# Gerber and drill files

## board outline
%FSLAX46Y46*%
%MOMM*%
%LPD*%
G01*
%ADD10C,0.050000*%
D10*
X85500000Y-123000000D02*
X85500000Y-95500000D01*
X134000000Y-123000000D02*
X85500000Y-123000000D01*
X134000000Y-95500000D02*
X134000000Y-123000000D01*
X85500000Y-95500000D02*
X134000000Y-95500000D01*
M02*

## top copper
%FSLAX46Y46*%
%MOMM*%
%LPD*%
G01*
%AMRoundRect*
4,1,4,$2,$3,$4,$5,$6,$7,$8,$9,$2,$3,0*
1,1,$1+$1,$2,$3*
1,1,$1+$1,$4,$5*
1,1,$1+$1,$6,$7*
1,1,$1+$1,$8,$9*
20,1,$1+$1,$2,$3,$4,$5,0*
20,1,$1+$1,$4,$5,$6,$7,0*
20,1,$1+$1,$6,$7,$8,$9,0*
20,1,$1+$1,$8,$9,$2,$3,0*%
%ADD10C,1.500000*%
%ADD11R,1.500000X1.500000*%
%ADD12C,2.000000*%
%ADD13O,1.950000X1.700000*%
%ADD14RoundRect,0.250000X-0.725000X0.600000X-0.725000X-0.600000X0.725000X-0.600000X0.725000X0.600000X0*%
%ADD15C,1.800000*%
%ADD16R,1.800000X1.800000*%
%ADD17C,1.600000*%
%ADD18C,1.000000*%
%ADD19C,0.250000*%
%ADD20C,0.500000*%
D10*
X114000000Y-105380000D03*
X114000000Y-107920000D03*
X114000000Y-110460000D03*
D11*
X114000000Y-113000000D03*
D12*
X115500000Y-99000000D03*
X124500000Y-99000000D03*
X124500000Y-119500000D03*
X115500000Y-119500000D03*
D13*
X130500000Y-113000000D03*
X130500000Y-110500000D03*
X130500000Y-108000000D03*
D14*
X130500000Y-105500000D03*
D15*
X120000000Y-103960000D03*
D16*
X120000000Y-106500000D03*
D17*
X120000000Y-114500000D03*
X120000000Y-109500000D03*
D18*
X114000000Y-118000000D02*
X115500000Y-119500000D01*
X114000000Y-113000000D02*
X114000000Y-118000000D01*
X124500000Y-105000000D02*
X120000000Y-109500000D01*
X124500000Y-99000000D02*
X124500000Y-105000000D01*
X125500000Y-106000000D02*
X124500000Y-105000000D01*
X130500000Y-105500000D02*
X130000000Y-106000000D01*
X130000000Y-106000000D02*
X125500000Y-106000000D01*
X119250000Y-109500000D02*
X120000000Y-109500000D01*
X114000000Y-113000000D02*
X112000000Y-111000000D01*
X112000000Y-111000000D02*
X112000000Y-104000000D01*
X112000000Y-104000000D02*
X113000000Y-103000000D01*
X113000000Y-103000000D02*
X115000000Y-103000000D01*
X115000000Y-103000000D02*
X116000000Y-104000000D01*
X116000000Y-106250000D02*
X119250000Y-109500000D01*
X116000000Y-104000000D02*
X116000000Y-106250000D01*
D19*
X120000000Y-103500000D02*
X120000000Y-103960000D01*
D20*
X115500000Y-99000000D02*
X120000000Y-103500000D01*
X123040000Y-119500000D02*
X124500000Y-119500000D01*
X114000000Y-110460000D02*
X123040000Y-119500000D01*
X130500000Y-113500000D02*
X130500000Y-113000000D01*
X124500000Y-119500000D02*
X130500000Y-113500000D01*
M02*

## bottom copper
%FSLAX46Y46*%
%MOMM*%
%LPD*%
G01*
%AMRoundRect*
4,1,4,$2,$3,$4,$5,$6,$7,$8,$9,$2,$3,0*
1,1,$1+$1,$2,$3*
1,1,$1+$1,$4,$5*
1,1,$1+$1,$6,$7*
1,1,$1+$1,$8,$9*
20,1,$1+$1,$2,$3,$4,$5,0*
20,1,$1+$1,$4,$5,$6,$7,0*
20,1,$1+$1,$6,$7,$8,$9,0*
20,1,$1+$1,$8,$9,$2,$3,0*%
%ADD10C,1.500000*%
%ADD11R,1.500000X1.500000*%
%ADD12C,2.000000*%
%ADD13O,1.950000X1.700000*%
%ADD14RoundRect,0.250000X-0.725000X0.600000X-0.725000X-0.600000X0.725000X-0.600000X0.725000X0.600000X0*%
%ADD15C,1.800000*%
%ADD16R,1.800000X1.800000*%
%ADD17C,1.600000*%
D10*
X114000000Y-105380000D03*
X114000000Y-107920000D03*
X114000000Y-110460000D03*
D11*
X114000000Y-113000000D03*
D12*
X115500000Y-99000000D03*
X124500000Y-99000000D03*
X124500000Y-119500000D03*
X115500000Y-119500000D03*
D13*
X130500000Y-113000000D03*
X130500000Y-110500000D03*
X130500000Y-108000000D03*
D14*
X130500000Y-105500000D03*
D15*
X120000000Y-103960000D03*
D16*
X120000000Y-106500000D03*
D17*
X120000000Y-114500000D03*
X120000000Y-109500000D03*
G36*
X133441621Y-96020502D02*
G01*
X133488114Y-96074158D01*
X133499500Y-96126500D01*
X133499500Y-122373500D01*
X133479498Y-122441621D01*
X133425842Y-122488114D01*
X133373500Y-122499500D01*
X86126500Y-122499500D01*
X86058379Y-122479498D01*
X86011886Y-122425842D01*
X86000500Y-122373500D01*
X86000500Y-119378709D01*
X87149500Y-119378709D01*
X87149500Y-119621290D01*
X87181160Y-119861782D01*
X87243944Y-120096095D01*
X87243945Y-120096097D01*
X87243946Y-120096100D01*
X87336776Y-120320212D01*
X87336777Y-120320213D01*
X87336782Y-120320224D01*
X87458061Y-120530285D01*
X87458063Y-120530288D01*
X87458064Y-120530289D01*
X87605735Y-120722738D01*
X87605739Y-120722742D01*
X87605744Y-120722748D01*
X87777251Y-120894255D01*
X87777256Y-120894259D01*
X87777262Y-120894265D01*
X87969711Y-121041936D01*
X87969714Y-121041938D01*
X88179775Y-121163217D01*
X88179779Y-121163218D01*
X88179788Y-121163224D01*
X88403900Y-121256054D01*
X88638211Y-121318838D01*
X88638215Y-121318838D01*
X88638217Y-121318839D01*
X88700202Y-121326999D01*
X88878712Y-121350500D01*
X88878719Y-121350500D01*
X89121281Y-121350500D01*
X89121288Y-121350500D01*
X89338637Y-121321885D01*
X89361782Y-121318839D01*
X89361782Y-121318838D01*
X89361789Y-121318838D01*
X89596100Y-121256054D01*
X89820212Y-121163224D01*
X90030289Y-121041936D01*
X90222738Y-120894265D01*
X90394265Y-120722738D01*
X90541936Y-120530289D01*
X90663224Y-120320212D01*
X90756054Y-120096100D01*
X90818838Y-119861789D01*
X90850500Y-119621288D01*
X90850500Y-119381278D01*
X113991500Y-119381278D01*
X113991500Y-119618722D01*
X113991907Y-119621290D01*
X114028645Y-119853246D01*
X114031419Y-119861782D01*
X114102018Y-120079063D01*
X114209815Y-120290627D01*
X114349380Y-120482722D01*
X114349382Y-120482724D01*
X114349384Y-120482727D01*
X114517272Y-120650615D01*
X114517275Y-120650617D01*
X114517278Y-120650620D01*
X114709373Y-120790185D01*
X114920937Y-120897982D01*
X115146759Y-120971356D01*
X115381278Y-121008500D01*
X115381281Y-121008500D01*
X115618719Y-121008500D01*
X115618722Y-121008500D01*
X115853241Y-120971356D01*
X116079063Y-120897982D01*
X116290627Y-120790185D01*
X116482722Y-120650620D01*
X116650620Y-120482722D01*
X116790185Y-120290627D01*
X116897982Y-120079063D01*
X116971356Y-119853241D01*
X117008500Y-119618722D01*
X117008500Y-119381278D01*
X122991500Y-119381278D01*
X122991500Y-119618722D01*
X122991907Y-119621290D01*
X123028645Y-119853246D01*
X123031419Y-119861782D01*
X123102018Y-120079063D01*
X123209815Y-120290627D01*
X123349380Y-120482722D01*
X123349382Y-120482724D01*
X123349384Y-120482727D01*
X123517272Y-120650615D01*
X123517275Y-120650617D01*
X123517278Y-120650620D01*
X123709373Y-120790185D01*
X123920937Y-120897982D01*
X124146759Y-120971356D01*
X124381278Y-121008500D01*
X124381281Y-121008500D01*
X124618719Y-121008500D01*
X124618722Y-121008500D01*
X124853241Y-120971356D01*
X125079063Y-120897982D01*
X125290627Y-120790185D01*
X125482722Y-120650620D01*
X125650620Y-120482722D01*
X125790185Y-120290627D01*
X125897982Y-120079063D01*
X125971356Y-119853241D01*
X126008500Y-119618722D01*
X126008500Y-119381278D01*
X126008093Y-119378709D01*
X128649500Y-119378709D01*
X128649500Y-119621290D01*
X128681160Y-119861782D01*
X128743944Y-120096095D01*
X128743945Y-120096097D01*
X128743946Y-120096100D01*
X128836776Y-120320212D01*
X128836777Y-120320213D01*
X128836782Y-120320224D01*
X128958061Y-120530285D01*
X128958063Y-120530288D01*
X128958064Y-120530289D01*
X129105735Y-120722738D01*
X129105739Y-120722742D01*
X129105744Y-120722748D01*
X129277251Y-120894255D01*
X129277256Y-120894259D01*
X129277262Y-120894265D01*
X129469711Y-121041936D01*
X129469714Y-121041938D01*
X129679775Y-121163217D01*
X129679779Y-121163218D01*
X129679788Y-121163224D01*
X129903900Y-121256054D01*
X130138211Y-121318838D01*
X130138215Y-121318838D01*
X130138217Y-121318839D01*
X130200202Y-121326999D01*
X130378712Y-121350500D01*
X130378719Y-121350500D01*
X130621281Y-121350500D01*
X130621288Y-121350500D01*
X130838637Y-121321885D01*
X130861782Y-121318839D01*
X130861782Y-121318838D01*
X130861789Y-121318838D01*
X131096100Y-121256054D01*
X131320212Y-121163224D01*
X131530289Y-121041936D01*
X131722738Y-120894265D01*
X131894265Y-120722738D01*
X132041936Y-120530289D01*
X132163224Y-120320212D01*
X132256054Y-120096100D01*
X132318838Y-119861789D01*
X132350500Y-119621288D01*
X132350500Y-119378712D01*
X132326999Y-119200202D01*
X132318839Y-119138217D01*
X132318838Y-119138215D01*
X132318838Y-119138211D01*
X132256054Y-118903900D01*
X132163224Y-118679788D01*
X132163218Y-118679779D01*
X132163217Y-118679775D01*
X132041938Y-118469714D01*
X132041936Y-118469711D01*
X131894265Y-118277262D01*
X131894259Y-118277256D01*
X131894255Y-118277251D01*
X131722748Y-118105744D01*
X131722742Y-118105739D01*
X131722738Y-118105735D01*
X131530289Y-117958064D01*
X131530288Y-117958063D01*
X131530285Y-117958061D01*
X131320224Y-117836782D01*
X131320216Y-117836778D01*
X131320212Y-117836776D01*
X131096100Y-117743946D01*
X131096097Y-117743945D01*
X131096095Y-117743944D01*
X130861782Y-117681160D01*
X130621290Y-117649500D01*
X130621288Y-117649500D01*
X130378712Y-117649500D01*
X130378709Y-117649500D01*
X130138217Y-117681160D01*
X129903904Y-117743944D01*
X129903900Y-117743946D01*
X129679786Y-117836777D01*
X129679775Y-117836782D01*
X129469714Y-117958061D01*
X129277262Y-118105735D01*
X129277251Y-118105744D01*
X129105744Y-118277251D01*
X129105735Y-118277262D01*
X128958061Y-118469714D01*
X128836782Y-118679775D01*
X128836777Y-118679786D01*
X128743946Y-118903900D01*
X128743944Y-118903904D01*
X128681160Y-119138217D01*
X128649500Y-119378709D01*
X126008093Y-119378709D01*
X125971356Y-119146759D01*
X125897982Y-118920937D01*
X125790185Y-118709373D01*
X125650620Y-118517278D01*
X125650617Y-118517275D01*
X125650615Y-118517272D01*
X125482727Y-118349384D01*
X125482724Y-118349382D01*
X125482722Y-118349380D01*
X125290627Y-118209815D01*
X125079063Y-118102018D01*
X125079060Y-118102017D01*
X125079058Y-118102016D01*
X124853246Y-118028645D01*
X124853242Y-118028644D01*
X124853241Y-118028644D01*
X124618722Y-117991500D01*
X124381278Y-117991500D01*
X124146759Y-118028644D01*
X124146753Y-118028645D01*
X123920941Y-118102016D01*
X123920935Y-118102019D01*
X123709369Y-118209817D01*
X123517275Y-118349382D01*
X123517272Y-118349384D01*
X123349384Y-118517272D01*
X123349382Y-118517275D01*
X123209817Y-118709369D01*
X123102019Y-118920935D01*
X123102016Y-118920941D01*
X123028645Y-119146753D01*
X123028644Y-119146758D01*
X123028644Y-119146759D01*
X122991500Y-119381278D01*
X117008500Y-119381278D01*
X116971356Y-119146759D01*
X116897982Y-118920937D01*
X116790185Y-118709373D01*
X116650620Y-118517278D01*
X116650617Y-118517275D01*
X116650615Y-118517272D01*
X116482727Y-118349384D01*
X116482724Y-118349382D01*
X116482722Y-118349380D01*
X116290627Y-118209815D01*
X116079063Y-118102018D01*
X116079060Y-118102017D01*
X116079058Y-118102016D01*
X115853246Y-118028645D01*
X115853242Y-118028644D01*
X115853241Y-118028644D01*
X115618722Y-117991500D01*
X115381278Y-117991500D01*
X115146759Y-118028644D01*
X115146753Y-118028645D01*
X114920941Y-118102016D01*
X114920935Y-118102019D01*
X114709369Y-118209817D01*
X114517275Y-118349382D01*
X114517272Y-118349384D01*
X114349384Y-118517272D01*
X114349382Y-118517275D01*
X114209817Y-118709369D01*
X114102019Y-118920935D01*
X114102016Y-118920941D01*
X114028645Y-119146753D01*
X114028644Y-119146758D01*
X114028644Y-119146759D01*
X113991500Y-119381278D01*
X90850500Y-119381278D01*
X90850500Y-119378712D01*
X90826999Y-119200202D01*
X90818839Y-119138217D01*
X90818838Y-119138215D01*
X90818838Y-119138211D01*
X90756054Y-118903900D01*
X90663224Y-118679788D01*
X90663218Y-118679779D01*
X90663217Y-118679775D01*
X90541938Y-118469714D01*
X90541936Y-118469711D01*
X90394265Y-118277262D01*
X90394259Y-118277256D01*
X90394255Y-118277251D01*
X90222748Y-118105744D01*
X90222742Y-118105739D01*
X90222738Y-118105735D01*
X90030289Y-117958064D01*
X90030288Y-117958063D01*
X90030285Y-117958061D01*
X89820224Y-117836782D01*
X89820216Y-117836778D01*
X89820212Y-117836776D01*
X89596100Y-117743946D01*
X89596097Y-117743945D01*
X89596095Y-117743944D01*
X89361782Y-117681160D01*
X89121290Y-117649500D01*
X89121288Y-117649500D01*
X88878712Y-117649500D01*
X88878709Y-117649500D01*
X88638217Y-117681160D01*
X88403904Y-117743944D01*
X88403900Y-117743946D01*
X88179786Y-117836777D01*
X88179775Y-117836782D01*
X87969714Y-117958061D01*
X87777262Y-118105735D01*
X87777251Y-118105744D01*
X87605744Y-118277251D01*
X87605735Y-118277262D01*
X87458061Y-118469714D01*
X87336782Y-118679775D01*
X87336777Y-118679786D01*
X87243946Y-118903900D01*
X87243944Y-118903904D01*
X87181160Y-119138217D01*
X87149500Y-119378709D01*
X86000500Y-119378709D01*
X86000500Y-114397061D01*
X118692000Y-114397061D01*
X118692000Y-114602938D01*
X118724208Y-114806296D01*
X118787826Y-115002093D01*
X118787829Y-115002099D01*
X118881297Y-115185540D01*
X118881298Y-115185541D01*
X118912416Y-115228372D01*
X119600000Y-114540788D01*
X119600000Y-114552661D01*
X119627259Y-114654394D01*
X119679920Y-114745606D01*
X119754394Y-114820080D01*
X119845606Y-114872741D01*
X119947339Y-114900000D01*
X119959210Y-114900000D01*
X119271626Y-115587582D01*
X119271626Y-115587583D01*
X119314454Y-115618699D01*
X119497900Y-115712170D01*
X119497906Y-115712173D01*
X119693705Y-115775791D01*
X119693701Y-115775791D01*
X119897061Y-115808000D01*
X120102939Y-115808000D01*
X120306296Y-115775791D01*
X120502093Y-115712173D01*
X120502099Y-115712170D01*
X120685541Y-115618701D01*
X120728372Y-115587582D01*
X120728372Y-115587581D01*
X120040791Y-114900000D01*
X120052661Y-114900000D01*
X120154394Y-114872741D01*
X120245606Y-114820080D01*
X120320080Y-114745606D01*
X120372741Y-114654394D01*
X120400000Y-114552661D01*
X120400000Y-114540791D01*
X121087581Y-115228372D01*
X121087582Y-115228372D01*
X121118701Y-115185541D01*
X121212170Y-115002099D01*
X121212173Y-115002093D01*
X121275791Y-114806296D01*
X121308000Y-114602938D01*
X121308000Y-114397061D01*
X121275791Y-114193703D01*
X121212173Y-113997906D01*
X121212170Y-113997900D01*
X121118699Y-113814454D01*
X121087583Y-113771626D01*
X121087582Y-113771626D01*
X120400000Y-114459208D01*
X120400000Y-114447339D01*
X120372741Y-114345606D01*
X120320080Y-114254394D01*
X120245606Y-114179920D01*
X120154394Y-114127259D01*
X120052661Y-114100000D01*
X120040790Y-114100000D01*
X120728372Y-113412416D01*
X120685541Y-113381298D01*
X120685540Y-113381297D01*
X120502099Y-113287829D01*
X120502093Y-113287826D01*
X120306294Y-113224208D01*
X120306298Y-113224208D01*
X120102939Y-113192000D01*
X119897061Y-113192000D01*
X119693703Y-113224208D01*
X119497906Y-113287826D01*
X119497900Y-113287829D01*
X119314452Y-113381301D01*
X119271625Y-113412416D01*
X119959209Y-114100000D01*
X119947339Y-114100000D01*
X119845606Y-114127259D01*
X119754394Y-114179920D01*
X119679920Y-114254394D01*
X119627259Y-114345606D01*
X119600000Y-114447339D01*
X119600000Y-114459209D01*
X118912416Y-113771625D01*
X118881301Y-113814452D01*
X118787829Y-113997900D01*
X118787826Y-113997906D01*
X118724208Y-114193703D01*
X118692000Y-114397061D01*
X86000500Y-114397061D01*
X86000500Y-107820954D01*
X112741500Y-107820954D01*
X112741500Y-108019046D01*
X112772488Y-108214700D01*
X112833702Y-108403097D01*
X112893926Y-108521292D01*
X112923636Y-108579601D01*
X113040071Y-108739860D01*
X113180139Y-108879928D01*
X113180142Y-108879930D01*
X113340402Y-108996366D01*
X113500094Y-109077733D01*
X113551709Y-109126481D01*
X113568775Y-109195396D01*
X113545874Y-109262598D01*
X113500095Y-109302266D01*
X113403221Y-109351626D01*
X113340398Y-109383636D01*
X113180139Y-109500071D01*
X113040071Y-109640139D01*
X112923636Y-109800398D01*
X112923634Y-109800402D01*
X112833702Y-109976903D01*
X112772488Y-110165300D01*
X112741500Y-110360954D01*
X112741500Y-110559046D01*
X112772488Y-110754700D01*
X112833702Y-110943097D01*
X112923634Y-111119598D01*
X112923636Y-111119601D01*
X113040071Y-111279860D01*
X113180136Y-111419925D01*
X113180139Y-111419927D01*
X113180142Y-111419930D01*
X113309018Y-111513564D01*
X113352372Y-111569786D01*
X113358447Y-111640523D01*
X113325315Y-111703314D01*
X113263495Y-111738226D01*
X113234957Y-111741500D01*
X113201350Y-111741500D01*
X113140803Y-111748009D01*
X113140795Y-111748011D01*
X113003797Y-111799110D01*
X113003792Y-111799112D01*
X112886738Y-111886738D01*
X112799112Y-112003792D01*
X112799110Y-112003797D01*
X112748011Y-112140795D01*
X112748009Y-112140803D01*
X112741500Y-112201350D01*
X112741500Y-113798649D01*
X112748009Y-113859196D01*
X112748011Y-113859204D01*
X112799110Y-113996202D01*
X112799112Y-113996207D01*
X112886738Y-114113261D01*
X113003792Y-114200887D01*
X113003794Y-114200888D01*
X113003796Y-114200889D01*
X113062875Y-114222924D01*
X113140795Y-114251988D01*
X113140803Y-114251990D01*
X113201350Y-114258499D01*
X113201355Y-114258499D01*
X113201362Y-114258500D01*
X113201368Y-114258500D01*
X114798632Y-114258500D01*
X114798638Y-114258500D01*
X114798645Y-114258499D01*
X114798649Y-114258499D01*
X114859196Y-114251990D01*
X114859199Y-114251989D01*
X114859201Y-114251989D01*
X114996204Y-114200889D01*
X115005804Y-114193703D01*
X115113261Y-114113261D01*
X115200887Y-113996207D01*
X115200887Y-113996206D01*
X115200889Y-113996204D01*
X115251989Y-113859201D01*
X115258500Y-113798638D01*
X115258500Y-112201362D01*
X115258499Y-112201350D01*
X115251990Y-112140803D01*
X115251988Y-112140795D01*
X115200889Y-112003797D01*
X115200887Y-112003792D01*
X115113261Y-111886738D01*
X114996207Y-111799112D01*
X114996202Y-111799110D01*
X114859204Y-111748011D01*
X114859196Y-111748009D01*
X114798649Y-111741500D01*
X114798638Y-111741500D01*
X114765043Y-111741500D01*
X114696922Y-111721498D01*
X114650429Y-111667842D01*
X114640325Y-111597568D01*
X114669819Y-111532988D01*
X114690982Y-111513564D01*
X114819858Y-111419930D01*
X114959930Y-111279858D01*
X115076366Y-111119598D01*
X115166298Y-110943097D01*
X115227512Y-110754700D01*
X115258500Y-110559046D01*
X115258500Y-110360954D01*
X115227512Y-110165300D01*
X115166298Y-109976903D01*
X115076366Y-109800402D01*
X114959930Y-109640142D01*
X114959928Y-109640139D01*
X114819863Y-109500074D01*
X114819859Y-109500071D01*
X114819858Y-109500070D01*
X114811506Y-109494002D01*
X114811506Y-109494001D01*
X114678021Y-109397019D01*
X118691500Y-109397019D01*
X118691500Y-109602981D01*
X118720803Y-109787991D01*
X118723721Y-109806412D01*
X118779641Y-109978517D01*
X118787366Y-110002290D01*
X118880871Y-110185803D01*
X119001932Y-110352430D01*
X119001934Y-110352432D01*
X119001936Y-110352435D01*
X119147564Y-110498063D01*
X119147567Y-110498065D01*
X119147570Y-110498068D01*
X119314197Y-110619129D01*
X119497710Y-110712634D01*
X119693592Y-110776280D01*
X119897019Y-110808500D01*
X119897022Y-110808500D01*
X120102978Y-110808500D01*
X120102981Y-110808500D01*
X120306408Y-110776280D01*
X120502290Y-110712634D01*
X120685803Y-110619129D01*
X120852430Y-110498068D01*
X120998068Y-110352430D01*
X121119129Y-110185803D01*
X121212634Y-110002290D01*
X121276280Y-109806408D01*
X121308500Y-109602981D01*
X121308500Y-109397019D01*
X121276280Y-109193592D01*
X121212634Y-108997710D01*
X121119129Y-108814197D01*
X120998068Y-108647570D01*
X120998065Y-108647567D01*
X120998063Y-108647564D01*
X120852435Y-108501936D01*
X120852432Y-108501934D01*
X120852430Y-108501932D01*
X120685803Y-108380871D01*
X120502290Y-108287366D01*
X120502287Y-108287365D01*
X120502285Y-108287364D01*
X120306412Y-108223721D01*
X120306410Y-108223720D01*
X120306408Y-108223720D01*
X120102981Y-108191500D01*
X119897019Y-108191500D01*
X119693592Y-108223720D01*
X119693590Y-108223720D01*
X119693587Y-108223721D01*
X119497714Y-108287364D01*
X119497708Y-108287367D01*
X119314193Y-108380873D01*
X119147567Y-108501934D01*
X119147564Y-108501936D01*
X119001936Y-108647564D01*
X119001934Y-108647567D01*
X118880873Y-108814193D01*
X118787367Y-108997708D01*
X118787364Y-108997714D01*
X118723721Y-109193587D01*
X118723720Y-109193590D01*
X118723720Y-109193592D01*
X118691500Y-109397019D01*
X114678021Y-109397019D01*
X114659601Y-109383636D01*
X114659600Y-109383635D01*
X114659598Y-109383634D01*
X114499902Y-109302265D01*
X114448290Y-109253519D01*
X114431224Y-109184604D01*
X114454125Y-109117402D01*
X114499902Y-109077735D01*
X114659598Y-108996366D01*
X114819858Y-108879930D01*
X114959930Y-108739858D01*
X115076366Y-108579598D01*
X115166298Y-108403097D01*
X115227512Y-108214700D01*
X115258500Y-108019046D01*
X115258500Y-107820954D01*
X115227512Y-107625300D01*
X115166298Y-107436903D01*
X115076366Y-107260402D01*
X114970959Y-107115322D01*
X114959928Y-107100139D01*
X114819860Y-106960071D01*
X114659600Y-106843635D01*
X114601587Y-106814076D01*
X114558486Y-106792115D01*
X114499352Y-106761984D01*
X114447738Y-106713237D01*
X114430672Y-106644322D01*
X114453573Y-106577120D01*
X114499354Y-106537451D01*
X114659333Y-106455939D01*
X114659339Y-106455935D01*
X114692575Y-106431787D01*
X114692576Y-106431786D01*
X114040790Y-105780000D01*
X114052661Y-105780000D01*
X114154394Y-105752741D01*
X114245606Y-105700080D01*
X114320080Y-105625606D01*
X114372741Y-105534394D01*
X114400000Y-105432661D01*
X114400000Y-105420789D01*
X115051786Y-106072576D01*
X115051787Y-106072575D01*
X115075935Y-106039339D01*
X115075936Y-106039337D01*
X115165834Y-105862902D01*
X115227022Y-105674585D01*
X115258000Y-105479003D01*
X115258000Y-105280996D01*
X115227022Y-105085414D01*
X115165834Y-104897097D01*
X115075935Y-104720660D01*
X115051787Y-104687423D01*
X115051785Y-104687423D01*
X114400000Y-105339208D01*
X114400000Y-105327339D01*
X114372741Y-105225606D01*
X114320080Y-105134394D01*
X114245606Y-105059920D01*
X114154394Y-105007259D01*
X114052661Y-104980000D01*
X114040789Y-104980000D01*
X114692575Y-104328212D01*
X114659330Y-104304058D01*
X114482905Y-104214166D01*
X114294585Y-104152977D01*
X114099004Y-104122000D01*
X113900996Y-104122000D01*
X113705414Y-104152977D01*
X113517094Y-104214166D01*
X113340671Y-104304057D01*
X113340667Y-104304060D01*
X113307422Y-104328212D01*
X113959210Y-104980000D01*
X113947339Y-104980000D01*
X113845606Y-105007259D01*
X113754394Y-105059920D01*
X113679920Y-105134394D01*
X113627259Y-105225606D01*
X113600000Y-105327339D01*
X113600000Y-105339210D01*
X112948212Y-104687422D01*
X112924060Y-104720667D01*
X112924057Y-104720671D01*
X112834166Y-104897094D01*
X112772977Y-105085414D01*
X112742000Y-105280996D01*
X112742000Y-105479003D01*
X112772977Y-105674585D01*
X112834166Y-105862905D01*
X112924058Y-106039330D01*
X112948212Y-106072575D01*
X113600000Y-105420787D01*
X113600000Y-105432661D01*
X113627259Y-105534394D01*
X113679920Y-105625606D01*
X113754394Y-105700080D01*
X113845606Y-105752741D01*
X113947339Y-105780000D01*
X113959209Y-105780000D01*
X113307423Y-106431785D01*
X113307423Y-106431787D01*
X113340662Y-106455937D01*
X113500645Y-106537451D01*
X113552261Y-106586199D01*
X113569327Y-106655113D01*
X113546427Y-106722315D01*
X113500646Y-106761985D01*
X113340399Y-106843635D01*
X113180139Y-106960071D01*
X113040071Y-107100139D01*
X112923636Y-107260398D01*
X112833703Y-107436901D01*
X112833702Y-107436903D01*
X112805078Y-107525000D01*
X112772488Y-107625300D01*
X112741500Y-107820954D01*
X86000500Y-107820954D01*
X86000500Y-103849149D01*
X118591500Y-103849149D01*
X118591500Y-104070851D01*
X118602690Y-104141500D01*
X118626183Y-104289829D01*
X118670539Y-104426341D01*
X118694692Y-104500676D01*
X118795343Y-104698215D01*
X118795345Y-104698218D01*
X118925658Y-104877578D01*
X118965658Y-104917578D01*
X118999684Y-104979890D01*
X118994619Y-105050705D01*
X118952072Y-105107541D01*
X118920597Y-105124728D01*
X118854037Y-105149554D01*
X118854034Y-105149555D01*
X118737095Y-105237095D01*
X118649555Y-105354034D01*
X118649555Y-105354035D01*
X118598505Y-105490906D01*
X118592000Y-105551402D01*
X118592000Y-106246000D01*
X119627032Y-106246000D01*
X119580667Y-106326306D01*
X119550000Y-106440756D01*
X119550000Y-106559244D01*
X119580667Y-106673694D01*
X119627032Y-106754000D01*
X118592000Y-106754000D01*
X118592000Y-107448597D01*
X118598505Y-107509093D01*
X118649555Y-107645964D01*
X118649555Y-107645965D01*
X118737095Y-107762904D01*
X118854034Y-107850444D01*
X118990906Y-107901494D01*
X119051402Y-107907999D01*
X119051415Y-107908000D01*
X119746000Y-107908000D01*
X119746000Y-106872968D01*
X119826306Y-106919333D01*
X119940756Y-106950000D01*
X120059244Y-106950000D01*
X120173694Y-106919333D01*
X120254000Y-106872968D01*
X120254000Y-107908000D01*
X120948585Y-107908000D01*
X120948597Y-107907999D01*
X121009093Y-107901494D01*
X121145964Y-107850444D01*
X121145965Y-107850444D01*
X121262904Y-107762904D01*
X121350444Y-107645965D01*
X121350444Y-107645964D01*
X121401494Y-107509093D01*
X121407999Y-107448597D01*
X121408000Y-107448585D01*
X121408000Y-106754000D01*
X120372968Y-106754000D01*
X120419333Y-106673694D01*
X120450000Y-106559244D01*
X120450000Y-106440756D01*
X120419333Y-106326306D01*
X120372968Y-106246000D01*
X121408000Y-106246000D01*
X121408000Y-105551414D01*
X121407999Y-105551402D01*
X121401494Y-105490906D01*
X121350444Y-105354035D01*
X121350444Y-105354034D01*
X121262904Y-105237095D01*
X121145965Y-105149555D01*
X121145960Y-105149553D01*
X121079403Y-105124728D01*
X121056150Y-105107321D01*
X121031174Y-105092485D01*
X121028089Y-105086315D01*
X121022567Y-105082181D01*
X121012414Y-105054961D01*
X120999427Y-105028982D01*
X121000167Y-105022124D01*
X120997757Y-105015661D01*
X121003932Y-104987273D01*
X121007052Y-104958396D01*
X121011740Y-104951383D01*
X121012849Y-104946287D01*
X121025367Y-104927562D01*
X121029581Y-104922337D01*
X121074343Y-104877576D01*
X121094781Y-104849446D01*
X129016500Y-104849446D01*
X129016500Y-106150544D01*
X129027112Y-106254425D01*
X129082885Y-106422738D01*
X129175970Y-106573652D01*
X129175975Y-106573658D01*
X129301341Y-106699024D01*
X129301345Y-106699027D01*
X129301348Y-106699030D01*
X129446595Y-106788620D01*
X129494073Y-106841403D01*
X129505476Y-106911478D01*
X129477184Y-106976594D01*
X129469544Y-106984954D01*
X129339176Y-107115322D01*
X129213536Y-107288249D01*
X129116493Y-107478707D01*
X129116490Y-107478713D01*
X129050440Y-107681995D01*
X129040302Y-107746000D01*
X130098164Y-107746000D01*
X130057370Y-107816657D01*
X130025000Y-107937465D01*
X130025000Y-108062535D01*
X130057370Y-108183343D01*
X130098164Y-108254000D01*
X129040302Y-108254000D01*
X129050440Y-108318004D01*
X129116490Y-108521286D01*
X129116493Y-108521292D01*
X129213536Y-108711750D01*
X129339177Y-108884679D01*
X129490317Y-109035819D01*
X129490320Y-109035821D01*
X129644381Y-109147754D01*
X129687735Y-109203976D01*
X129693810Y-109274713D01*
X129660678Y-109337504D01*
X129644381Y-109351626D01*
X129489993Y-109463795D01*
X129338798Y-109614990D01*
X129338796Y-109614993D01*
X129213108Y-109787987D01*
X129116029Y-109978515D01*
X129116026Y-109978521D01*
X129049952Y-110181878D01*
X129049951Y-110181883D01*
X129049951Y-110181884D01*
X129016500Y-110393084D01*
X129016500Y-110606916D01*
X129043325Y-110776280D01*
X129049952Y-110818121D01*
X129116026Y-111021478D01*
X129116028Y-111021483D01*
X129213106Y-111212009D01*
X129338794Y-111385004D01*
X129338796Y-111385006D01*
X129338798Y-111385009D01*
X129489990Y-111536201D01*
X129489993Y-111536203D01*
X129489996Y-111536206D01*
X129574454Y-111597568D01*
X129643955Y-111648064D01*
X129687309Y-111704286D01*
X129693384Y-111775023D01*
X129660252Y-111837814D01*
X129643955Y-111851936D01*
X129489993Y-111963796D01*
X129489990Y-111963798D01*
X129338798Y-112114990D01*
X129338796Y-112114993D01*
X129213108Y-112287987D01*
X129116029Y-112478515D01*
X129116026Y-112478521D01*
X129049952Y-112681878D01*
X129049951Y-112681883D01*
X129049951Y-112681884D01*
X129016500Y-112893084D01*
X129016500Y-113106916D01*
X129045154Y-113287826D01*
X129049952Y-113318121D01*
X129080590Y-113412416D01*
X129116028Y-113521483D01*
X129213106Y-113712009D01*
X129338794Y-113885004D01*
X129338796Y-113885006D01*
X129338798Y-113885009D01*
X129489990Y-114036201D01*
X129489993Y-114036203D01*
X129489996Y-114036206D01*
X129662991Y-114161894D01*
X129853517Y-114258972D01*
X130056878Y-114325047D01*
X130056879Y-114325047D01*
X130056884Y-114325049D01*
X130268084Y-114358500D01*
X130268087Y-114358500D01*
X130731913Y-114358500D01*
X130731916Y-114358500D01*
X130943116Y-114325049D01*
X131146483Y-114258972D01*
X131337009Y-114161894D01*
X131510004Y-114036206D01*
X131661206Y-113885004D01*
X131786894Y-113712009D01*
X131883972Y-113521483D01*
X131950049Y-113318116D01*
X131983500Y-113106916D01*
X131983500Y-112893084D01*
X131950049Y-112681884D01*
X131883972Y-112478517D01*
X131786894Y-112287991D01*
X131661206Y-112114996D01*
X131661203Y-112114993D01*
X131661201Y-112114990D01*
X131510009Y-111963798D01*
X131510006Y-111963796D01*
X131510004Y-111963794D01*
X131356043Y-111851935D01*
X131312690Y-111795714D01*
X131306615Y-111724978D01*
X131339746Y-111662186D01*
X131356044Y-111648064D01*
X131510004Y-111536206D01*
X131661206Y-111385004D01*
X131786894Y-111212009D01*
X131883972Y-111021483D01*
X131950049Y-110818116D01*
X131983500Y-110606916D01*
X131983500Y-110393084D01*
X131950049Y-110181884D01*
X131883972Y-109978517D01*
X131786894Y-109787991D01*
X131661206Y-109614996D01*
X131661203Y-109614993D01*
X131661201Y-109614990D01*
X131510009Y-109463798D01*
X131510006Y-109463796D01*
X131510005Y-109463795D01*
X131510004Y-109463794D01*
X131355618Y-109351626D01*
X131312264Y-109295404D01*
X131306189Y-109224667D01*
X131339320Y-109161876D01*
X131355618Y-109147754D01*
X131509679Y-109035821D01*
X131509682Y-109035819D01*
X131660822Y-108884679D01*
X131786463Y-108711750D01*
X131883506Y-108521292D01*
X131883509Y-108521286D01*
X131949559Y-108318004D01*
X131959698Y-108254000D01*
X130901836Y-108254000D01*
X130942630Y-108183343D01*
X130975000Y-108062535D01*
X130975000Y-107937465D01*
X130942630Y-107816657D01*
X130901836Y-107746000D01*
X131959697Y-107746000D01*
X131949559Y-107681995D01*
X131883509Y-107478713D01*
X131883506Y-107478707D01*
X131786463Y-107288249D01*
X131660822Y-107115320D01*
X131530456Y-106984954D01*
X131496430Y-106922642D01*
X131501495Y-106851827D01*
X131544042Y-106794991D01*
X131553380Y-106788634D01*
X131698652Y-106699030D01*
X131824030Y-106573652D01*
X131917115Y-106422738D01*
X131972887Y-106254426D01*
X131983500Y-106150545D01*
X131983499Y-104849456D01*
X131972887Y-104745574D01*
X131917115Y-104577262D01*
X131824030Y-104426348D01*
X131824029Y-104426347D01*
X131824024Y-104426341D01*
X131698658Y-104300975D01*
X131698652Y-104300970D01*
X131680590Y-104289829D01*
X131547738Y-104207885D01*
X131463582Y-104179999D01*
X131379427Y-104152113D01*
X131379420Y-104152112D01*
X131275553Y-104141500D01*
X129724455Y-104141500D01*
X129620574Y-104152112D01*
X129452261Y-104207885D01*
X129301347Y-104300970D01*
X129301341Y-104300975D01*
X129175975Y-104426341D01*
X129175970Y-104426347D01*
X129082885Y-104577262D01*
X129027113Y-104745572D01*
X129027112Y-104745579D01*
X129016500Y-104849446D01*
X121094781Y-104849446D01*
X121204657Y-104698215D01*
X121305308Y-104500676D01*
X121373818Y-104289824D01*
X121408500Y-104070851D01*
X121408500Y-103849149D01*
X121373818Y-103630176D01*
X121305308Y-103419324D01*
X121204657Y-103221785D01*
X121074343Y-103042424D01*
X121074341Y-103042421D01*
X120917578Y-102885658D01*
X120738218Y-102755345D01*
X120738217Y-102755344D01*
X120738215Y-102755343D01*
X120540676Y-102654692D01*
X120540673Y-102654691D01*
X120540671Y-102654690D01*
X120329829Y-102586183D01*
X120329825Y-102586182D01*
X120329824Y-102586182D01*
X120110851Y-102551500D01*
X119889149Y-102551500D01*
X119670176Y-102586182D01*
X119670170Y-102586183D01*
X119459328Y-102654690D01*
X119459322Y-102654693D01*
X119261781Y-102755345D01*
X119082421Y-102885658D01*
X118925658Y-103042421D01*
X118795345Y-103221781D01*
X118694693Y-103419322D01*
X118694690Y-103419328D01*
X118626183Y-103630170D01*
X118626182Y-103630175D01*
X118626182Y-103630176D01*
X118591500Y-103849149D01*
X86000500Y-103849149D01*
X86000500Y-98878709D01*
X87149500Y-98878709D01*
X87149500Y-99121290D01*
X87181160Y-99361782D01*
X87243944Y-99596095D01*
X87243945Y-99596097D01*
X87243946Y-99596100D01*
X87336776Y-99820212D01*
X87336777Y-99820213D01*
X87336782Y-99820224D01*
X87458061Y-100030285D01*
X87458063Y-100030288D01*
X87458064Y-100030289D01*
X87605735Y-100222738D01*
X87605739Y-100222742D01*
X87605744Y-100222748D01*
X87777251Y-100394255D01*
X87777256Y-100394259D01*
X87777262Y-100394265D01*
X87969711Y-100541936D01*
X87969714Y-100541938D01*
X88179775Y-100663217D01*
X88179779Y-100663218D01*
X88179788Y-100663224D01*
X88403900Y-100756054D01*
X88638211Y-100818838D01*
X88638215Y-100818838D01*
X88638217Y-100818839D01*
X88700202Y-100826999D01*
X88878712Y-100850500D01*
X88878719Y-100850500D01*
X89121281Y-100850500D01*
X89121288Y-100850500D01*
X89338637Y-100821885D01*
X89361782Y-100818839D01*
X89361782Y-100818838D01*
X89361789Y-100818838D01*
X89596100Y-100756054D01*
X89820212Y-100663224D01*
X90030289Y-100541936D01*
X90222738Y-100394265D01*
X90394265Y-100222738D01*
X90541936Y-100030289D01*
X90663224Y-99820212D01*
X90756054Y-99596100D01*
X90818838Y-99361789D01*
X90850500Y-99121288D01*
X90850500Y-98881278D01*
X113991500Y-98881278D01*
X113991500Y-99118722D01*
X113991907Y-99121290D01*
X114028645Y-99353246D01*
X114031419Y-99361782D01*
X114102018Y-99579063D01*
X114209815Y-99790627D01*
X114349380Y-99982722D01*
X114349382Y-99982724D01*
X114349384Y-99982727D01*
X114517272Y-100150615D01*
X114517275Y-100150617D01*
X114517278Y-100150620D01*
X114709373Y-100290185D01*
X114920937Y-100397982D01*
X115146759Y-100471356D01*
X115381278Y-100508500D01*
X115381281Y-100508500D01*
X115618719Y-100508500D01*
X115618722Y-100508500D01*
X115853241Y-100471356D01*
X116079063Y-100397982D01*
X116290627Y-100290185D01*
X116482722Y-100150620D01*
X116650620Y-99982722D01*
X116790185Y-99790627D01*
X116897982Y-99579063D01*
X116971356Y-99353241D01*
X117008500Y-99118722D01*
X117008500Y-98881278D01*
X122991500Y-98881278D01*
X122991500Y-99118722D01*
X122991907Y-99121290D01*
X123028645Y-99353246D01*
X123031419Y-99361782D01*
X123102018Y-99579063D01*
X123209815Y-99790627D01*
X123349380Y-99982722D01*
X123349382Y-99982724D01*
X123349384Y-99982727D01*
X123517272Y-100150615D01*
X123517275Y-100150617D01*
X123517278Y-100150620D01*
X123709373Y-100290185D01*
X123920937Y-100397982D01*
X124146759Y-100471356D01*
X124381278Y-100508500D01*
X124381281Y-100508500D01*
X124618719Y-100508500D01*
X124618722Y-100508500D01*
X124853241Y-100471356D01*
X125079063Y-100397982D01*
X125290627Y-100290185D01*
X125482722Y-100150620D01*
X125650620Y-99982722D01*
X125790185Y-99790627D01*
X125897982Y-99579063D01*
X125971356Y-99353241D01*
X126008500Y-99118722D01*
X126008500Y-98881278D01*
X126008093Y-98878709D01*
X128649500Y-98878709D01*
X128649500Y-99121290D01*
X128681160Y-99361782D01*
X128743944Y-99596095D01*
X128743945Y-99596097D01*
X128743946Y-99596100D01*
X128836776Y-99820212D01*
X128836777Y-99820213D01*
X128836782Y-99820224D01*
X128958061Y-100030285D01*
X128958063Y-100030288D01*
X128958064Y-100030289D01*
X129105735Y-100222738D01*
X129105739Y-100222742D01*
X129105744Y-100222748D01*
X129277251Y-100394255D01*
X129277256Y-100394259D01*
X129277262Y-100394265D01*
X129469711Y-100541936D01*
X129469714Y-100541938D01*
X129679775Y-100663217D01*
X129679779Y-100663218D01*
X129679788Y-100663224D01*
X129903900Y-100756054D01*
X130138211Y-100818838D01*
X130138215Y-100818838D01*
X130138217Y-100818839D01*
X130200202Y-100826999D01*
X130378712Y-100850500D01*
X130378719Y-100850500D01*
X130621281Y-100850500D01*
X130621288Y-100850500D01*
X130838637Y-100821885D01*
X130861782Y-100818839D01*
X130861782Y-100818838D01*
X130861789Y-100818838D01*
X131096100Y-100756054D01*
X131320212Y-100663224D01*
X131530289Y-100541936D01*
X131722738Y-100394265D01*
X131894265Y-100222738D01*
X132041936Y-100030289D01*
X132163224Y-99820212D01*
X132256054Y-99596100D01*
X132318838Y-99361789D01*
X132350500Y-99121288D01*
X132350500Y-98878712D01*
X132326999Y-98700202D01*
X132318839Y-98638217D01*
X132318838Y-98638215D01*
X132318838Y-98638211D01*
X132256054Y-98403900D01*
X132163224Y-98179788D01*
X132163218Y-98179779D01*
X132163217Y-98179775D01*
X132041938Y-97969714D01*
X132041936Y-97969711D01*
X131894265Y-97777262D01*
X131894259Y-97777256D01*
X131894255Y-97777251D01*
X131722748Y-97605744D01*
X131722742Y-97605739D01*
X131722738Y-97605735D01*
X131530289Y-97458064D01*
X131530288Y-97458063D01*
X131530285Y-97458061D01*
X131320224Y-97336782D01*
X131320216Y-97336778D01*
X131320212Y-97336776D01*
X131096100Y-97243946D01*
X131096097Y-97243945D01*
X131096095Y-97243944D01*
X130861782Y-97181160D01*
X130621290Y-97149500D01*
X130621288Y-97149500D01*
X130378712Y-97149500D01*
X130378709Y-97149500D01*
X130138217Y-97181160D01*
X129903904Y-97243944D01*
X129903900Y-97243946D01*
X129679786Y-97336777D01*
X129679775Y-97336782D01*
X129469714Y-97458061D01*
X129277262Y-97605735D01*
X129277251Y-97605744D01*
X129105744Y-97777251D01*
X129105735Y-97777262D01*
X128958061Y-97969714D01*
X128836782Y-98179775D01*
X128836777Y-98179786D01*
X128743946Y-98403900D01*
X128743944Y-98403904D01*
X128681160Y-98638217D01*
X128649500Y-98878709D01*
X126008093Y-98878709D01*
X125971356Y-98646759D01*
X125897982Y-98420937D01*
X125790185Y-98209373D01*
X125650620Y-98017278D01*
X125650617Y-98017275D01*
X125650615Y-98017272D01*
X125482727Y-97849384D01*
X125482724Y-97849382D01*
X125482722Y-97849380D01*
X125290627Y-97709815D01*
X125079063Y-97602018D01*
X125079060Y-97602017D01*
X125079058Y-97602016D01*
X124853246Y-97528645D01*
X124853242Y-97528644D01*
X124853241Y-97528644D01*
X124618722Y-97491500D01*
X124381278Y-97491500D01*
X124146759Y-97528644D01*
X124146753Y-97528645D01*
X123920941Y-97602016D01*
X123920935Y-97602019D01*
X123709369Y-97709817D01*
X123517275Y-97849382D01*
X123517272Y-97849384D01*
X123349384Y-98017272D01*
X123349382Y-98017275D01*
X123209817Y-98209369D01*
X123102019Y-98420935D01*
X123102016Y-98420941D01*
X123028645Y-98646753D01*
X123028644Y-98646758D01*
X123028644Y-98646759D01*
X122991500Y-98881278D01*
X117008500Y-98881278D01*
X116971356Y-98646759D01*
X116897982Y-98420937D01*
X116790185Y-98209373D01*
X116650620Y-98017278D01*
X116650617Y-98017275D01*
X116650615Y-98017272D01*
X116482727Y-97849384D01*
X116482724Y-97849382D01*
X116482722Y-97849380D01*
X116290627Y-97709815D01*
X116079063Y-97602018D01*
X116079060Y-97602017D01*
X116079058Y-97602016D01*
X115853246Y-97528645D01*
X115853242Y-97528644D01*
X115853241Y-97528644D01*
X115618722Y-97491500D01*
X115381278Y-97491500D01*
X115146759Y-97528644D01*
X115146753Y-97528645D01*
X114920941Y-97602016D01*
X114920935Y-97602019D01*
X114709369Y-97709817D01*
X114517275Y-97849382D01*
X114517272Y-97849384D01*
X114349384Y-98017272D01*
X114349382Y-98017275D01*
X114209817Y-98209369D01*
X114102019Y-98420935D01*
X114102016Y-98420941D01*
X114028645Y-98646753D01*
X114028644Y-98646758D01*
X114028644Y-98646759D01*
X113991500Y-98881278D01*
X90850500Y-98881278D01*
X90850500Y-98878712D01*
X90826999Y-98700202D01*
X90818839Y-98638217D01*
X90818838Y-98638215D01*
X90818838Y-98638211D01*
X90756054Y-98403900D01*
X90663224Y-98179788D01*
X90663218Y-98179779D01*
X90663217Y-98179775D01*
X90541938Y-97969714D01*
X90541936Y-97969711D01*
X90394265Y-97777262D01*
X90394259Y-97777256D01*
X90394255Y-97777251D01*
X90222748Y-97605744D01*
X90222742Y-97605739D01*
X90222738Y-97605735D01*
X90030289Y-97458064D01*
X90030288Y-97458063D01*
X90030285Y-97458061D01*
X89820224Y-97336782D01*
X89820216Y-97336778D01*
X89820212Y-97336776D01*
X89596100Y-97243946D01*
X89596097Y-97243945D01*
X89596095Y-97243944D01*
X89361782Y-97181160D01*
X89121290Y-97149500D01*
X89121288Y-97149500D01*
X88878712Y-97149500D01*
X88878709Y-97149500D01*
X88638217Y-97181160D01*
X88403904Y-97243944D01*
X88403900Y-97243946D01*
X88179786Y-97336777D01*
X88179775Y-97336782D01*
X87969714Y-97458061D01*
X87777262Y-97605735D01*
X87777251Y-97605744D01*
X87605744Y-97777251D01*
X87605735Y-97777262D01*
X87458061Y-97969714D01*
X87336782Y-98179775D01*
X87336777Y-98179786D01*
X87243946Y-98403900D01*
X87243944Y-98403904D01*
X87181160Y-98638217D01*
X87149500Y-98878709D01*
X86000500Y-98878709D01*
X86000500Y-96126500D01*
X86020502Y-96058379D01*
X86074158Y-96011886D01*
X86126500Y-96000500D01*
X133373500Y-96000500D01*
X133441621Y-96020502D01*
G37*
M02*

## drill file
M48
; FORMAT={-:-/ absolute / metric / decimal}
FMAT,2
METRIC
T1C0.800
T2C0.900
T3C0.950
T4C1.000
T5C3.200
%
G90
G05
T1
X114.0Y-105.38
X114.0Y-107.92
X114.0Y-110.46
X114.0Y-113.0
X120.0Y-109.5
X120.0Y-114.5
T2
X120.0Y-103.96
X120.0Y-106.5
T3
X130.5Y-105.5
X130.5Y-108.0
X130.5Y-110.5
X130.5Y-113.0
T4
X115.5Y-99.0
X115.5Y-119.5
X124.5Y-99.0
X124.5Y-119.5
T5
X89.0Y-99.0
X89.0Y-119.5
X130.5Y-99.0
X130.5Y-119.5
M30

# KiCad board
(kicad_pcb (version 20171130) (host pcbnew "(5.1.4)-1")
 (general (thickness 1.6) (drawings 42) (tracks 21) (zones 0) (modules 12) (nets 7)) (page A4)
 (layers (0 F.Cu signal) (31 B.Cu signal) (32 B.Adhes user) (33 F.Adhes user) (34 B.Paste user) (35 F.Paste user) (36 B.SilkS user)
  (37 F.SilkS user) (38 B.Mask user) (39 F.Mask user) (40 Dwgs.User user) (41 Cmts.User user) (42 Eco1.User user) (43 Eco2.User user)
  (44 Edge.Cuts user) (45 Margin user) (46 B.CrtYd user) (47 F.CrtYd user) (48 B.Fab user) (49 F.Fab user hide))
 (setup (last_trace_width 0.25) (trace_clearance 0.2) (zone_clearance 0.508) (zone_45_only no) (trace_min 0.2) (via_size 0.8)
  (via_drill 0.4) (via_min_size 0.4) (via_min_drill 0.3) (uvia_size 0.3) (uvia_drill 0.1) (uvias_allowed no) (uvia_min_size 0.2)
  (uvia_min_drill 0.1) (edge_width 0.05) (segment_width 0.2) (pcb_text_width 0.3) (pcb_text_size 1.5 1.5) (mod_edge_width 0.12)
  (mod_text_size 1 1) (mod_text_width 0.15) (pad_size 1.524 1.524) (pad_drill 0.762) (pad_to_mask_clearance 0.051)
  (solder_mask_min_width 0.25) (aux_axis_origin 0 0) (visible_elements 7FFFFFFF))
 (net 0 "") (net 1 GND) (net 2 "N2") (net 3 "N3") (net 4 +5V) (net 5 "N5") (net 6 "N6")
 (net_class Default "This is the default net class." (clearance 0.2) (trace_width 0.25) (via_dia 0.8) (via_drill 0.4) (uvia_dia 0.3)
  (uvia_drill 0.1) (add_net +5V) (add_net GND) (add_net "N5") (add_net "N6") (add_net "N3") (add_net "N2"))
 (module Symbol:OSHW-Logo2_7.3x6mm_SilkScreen (layer F.Cu) (at 102 119.5)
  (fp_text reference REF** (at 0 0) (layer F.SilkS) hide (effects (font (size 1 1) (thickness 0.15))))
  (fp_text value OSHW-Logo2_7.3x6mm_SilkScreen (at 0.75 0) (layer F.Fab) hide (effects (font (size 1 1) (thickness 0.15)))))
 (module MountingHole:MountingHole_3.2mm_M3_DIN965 (layer F.Cu) (at 89 119.5 180)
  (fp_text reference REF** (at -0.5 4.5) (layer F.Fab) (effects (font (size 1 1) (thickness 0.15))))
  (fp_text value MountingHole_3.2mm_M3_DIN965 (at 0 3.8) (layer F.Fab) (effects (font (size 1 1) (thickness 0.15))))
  (pad 1 np_thru_hole circle (at 0 0 180) (size 3.2 3.2) (drill 3.2) (layers *.Cu *.Mask)))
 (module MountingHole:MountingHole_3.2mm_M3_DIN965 (layer F.Cu) (at 89 99 90)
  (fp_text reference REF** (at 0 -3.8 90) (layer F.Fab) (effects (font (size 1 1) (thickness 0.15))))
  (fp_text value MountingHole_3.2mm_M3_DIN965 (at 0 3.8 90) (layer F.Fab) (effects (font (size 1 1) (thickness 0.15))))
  (pad 1 np_thru_hole circle (at 0 0 90) (size 3.2 3.2) (drill 3.2) (layers *.Cu *.Mask)))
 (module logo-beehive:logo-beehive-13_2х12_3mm (layer B.Cu) (at 122.5 109.5 270)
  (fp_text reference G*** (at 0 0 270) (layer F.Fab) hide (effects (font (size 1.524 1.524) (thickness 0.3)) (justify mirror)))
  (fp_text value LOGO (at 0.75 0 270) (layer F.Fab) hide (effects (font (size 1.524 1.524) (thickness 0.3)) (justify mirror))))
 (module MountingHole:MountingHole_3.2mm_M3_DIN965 (layer F.Cu) (at 130.5 119.5)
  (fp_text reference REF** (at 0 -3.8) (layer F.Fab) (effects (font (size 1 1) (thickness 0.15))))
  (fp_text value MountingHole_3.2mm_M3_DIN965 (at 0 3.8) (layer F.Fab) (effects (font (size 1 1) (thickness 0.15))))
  (pad 1 np_thru_hole circle (at 0 0) (size 3.2 3.2) (drill 3.2) (layers *.Cu *.Mask)))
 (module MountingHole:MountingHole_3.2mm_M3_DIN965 (layer F.Cu) (at 130.5 99)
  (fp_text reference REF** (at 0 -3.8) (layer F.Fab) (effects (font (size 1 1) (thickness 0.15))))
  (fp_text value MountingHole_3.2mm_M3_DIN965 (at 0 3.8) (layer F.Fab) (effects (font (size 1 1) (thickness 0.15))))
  (pad 1 np_thru_hole circle (at 0 0) (size 3.2 3.2) (drill 3.2) (layers *.Cu *.Mask)))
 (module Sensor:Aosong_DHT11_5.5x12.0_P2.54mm (layer F.Cu) (at 114 113 180)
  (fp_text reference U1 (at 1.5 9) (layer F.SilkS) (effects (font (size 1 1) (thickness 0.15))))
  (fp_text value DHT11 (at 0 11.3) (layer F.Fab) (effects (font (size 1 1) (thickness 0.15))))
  (pad 4 thru_hole circle (at 0 7.62 180) (size 1.5 1.5) (drill 0.8) (layers *.Cu *.Mask) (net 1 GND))
  (pad 3 thru_hole circle (at 0 5.08 180) (size 1.5 1.5) (drill 0.8) (layers *.Cu *.Mask) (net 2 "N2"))
  (pad 2 thru_hole circle (at 0 2.54 180) (size 1.5 1.5) (drill 0.8) (layers *.Cu *.Mask) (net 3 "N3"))
  (pad 1 thru_hole rect (at 0 0 180) (size 1.5 1.5) (drill 0.8) (layers *.Cu *.Mask) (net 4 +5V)))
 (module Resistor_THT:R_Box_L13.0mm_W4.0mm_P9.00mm (layer F.Cu) (at 124.5 99 180)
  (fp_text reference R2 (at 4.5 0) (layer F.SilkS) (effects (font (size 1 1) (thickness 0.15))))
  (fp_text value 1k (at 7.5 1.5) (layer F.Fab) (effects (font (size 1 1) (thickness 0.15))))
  (pad 2 thru_hole circle (at 9 0 180) (size 2 2) (drill 1) (layers *.Cu *.Mask) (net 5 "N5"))
  (pad 1 thru_hole circle (at 0 0 180) (size 2 2) (drill 1) (layers *.Cu *.Mask) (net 4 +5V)))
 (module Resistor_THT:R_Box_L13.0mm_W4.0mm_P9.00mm (layer F.Cu) (at 115.5 119.5)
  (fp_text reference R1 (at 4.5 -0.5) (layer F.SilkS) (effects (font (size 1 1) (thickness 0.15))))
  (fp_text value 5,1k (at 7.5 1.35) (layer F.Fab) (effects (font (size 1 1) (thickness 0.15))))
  (pad 2 thru_hole circle (at 9 0) (size 2 2) (drill 1) (layers *.Cu *.Mask) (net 3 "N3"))
  (pad 1 thru_hole circle (at 0 0) (size 2 2) (drill 1) (layers *.Cu *.Mask) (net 4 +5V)))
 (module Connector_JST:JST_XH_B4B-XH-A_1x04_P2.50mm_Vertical (layer F.Cu) (at 130.5 105.5 270)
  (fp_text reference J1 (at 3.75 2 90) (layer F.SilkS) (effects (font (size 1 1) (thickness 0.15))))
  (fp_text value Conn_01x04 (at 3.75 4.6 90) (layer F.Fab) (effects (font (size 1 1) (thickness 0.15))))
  (pad 4 thru_hole oval (at 7.5 0 270) (size 1.7 1.95) (drill 0.95) (layers *.Cu *.Mask) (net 3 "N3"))
  (pad 3 thru_hole oval (at 5 0 270) (size 1.7 1.95) (drill 0.95) (layers *.Cu *.Mask) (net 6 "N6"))
  (pad 2 thru_hole oval (at 2.5 0 270) (size 1.7 1.95) (drill 0.95) (layers *.Cu *.Mask) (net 1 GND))
  (pad 1 thru_hole roundrect (at 0 0 270) (size 1.7 1.95) (drill 0.95) (layers *.Cu *.Mask) (roundrect_rratio 0.147059) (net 4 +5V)))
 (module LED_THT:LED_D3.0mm (layer F.Cu) (at 120 106.5 90)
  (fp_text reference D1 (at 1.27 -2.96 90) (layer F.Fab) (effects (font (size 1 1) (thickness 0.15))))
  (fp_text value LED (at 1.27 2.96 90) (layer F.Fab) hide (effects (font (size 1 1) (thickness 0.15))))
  (pad 2 thru_hole circle (at 2.54 0 90) (size 1.8 1.8) (drill 0.9) (layers *.Cu *.Mask) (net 5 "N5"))
  (pad 1 thru_hole rect (at 0 0 90) (size 1.8 1.8) (drill 0.9) (layers *.Cu *.Mask) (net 1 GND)))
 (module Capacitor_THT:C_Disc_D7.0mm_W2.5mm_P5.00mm (layer F.Cu) (at 120 109.5 270)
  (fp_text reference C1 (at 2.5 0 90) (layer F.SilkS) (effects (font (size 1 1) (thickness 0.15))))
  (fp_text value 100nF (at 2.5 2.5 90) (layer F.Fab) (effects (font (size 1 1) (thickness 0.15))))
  (pad 2 thru_hole circle (at 5 0 270) (size 1.6 1.6) (drill 0.8) (layers *.Cu *.Mask) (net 1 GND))
  (pad 1 thru_hole circle (at 0 0 270) (size 1.6 1.6) (drill 0.8) (layers *.Cu *.Mask) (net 4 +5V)))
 (gr_line (start 85.5 123) (end 85.5 95.5) (layer Edge.Cuts) (width 0.05))
 (gr_line (start 134 123) (end 85.5 123) (layer Edge.Cuts) (width 0.05))
 (gr_line (start 134 95.5) (end 134 123) (layer Edge.Cuts) (width 0.05))
 (gr_line (start 85.5 95.5) (end 134 95.5) (layer Edge.Cuts) (width 0.05))
 (segment (start 114 118) (end 115.5 119.5) (width 1) (layer F.Cu) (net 4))
 (segment (start 114 113) (end 114 118) (width 1) (layer F.Cu) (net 4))
 (segment (start 124.5 105) (end 120 109.5) (width 1) (layer F.Cu) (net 4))
 (segment (start 124.5 99) (end 124.5 105) (width 1) (layer F.Cu) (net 4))
 (segment (start 125.5 106) (end 124.5 105) (width 1) (layer F.Cu) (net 4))
 (segment (start 130.5 105.5) (end 130 106) (width 1) (layer F.Cu) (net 4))
 (segment (start 130 106) (end 125.5 106) (width 1) (layer F.Cu) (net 4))
 (segment (start 119.25 109.5) (end 120 109.5) (width 1) (layer F.Cu) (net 4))
 (segment (start 114 113) (end 112 111) (width 1) (layer F.Cu) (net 4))
 (segment (start 112 111) (end 112 104) (width 1) (layer F.Cu) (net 4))
 (segment (start 112 104) (end 113 103) (width 1) (layer F.Cu) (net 4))
 (segment (start 113 103) (end 115 103) (width 1) (layer F.Cu) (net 4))
 (segment (start 115 103) (end 116 104) (width 1) (layer F.Cu) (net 4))
 (segment (start 116 106.25) (end 119.25 109.5) (width 1) (layer F.Cu) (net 4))
 (segment (start 116 104) (end 116 106.25) (width 1) (layer F.Cu) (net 4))
 (segment (start 120 103.5) (end 120 103.96) (width 0.25) (layer F.Cu) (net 5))
 (segment (start 115.5 99) (end 120 103.5) (width 0.5) (layer F.Cu) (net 5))
 (segment (start 123.04 119.5) (end 124.5 119.5) (width 0.5) (layer F.Cu) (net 3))
 (segment (start 114 110.46) (end 123.04 119.5) (width 0.5) (layer F.Cu) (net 3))
 (segment (start 130.5 113.5) (end 130.5 113) (width 0.5) (layer F.Cu) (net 3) (status 1000000))
 (segment (start 124.5 119.5) (end 130.5 113.5) (width 0.5) (layer F.Cu) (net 3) (status 1000000))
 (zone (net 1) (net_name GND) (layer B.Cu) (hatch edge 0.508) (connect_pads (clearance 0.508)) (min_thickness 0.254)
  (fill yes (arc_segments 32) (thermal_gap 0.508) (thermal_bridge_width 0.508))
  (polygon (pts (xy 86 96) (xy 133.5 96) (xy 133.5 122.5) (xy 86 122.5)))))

